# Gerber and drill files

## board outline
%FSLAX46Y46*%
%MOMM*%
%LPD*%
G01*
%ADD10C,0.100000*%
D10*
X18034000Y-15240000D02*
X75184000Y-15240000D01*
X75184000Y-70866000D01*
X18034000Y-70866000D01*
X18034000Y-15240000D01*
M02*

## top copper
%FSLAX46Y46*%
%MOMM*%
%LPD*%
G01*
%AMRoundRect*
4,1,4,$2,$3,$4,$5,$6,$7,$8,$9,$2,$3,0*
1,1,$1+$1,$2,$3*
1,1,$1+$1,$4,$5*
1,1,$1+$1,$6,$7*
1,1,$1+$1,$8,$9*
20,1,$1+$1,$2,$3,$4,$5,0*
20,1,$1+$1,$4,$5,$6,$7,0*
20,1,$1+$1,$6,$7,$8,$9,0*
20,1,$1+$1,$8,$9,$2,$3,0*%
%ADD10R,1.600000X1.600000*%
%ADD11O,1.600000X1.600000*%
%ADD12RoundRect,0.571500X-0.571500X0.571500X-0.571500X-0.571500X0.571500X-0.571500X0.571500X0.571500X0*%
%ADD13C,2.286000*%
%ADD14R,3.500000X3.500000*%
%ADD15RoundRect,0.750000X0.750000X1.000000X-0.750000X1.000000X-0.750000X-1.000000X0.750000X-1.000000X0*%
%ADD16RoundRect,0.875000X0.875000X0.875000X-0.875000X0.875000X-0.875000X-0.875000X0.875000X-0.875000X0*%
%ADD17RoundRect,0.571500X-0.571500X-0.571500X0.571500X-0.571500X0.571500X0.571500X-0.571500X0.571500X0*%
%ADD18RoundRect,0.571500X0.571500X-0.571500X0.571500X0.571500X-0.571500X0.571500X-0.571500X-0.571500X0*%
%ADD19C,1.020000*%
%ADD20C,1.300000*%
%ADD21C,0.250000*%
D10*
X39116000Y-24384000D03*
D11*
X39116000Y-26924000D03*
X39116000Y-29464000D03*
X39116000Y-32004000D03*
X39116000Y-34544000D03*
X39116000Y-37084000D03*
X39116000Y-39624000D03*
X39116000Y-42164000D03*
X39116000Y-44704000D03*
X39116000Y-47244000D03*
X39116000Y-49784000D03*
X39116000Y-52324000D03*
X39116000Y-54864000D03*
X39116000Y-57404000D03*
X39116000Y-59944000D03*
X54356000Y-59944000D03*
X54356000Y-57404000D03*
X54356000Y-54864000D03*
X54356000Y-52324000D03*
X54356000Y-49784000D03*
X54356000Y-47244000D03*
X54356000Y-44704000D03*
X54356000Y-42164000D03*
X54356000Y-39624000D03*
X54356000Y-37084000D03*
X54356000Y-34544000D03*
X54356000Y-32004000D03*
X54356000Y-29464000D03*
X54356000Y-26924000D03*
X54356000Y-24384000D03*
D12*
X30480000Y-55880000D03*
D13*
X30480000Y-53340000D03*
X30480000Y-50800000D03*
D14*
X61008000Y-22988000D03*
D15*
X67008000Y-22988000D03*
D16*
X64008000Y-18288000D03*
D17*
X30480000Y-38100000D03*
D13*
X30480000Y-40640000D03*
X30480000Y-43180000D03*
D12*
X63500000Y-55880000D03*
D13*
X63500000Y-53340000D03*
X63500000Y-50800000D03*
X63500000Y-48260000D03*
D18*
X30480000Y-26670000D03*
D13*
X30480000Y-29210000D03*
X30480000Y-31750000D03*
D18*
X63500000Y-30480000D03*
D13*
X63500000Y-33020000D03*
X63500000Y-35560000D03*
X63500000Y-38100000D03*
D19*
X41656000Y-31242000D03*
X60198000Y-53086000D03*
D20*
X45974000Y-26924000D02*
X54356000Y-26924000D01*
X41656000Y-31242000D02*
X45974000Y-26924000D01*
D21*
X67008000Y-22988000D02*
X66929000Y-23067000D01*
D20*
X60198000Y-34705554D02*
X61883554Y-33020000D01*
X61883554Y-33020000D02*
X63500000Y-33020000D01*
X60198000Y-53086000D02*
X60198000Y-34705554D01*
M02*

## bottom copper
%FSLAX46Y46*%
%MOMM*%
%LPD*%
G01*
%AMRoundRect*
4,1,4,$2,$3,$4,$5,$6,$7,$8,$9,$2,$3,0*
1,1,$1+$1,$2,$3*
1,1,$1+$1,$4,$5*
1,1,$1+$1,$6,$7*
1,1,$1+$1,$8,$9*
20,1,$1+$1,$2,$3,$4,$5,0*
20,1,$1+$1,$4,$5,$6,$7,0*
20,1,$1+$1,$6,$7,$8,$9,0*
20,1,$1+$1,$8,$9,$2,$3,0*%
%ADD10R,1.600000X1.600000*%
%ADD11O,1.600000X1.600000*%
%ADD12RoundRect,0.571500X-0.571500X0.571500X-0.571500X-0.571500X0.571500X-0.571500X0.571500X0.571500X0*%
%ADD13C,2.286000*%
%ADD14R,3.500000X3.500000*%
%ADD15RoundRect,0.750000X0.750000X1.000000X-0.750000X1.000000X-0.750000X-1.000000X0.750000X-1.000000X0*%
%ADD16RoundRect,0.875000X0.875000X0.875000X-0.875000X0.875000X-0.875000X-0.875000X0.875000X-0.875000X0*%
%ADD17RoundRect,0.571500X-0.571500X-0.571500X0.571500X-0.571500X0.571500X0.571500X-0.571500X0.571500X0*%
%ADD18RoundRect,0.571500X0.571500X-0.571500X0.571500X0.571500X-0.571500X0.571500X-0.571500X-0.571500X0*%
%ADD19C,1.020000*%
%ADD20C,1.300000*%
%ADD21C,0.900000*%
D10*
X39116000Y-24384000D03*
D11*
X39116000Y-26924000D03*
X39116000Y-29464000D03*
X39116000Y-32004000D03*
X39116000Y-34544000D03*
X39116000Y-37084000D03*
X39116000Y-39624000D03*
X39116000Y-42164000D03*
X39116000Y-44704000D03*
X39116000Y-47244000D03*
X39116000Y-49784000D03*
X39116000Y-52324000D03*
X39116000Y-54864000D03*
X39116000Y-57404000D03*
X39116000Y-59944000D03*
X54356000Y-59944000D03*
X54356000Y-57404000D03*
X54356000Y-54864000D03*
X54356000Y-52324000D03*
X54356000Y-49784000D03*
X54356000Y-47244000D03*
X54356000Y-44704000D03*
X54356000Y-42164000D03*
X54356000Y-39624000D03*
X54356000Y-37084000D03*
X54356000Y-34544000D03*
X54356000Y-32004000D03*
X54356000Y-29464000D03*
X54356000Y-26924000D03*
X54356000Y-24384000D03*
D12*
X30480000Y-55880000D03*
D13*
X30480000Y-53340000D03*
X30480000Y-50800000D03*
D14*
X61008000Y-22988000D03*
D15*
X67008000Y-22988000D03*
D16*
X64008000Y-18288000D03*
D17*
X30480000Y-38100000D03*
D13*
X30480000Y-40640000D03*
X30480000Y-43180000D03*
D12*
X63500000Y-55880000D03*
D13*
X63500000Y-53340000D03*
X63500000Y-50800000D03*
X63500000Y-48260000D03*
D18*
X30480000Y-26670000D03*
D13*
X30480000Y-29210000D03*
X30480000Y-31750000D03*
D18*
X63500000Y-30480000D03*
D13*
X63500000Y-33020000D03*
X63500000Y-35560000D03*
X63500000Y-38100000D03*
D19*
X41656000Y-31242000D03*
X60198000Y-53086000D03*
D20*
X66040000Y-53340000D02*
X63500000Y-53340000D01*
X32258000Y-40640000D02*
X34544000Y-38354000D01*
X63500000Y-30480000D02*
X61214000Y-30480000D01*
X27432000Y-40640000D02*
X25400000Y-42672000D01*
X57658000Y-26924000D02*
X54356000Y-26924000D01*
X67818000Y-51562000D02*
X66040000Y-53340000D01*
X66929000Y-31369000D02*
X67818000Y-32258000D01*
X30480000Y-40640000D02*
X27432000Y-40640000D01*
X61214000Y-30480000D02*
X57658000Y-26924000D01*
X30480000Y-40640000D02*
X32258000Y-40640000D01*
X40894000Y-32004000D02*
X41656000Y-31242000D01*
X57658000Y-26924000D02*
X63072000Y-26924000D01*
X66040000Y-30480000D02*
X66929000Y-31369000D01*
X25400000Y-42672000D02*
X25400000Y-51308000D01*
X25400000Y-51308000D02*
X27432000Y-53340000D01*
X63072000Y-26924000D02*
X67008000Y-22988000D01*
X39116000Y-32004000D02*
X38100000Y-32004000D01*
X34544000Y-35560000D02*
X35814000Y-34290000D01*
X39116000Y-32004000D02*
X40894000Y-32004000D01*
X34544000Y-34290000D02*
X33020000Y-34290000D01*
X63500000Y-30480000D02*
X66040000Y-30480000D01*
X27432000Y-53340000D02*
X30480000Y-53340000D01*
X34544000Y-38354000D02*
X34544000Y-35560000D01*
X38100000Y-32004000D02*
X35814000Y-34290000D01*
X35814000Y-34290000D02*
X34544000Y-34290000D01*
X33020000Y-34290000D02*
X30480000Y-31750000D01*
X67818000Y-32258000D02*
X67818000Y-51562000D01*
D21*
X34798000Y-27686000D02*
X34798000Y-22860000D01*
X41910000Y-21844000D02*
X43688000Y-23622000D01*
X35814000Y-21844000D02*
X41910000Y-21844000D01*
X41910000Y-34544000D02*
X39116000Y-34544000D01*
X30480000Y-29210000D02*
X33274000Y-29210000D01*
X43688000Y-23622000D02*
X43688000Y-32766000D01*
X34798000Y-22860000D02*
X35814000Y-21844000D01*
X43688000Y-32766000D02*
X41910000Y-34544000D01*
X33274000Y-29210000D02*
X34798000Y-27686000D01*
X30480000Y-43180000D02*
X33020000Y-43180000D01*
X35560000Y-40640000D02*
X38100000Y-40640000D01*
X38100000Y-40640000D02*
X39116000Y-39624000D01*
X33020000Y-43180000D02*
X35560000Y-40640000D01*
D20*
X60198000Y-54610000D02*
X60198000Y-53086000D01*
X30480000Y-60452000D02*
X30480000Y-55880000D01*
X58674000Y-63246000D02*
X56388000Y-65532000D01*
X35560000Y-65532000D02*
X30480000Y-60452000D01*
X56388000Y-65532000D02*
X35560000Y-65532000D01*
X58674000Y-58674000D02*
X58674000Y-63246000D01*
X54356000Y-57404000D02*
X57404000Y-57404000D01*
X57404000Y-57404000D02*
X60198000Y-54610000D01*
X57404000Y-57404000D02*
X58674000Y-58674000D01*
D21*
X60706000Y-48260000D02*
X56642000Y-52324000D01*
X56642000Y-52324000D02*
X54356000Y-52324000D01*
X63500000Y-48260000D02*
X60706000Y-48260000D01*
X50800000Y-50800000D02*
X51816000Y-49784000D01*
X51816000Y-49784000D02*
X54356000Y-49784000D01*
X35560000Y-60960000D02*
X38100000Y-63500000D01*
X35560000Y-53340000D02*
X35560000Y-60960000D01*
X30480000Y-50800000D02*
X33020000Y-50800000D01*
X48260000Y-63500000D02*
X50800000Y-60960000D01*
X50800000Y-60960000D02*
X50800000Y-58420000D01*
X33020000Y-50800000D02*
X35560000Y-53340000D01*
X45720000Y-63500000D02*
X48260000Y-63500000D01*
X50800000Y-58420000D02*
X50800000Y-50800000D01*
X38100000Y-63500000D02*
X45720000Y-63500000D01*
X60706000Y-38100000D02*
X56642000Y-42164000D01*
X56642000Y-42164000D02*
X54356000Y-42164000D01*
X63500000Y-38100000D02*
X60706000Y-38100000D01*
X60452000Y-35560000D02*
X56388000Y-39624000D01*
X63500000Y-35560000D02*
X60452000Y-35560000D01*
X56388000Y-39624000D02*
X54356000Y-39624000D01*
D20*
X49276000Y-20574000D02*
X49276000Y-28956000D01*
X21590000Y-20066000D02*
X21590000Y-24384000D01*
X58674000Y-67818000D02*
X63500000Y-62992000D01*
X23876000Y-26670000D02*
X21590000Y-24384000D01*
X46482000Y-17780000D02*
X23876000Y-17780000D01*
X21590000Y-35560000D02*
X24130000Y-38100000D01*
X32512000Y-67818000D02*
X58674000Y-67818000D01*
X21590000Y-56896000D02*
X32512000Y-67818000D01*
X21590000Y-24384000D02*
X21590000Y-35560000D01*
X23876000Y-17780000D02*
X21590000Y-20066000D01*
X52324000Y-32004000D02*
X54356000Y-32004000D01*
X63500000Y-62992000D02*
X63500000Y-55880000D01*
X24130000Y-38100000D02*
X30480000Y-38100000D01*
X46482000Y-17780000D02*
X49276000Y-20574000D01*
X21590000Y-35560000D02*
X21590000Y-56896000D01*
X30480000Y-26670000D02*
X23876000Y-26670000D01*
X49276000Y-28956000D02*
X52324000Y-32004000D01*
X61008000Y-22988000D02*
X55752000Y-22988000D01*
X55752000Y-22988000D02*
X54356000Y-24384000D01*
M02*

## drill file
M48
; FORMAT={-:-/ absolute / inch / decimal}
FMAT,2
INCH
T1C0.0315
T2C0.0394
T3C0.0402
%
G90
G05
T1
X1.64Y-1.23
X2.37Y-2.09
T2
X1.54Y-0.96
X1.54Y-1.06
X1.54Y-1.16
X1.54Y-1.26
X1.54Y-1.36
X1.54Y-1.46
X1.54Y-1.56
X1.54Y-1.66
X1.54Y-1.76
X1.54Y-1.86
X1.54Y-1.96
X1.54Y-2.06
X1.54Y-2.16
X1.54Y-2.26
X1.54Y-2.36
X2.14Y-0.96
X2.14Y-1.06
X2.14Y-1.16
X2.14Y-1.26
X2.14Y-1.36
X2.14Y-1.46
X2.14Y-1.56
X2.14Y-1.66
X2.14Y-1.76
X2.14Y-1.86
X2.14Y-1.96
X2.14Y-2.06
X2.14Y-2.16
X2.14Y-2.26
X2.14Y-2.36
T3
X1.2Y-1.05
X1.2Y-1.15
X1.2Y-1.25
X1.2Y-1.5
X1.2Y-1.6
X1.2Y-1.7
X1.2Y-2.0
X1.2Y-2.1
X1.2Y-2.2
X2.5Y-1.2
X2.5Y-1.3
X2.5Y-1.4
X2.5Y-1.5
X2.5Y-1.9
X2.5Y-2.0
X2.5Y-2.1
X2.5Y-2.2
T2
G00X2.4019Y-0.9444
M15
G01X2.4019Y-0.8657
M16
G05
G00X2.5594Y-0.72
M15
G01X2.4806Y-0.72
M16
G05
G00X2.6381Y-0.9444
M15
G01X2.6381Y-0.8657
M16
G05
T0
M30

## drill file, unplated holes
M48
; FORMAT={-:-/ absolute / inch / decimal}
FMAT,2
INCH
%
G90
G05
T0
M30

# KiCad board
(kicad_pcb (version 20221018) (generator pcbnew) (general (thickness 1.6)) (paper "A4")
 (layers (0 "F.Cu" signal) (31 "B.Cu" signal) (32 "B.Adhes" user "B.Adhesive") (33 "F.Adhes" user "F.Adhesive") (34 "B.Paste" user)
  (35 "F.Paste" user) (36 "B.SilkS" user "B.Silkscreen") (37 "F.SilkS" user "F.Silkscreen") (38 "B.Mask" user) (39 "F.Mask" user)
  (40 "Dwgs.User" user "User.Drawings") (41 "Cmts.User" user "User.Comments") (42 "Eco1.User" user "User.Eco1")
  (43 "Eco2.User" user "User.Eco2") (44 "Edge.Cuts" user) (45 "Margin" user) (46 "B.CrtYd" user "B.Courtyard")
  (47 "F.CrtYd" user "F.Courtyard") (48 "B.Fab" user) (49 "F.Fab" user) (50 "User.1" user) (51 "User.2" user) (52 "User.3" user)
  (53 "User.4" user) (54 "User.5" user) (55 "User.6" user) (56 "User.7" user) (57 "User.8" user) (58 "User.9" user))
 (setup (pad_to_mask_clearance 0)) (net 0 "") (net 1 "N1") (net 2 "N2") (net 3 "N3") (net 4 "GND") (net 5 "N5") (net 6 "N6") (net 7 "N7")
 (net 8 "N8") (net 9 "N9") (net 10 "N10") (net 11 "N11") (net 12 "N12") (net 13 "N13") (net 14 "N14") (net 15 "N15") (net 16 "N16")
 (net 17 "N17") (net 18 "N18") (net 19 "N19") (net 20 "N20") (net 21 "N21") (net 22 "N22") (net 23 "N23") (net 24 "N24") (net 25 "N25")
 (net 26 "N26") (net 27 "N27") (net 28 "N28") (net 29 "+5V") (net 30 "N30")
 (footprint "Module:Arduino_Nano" (layer "F.Cu") (at 39.116 24.384)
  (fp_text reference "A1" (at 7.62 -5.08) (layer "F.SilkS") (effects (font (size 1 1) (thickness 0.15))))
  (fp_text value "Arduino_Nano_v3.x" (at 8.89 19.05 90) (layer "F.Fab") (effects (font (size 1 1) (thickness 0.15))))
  (pad "1" thru_hole rect (at 0 0) (size 1.6 1.6) (drill 1) (layers "*.Cu" "*.Mask") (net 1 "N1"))
  (pad "2" thru_hole oval (at 0 2.54) (size 1.6 1.6) (drill 1) (layers "*.Cu" "*.Mask") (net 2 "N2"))
  (pad "3" thru_hole oval (at 0 5.08) (size 1.6 1.6) (drill 1) (layers "*.Cu" "*.Mask") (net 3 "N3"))
  (pad "4" thru_hole oval (at 0 7.62) (size 1.6 1.6) (drill 1) (layers "*.Cu" "*.Mask") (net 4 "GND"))
  (pad "5" thru_hole oval (at 0 10.16) (size 1.6 1.6) (drill 1) (layers "*.Cu" "*.Mask") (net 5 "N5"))
  (pad "6" thru_hole oval (at 0 12.7) (size 1.6 1.6) (drill 1) (layers "*.Cu" "*.Mask") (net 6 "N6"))
  (pad "7" thru_hole oval (at 0 15.24) (size 1.6 1.6) (drill 1) (layers "*.Cu" "*.Mask") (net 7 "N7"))
  (pad "8" thru_hole oval (at 0 17.78) (size 1.6 1.6) (drill 1) (layers "*.Cu" "*.Mask") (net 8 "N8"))
  (pad "9" thru_hole oval (at 0 20.32) (size 1.6 1.6) (drill 1) (layers "*.Cu" "*.Mask") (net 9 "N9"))
  (pad "10" thru_hole oval (at 0 22.86) (size 1.6 1.6) (drill 1) (layers "*.Cu" "*.Mask") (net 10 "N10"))
  (pad "11" thru_hole oval (at 0 25.4) (size 1.6 1.6) (drill 1) (layers "*.Cu" "*.Mask") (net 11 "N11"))
  (pad "12" thru_hole oval (at 0 27.94) (size 1.6 1.6) (drill 1) (layers "*.Cu" "*.Mask") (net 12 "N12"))
  (pad "13" thru_hole oval (at 0 30.48) (size 1.6 1.6) (drill 1) (layers "*.Cu" "*.Mask") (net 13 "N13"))
  (pad "14" thru_hole oval (at 0 33.02) (size 1.6 1.6) (drill 1) (layers "*.Cu" "*.Mask") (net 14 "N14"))
  (pad "15" thru_hole oval (at 0 35.56) (size 1.6 1.6) (drill 1) (layers "*.Cu" "*.Mask") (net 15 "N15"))
  (pad "16" thru_hole oval (at 15.24 35.56) (size 1.6 1.6) (drill 1) (layers "*.Cu" "*.Mask") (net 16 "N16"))
  (pad "17" thru_hole oval (at 15.24 33.02) (size 1.6 1.6) (drill 1) (layers "*.Cu" "*.Mask") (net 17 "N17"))
  (pad "18" thru_hole oval (at 15.24 30.48) (size 1.6 1.6) (drill 1) (layers "*.Cu" "*.Mask") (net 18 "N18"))
  (pad "19" thru_hole oval (at 15.24 27.94) (size 1.6 1.6) (drill 1) (layers "*.Cu" "*.Mask") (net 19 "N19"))
  (pad "20" thru_hole oval (at 15.24 25.4) (size 1.6 1.6) (drill 1) (layers "*.Cu" "*.Mask") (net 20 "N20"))
  (pad "21" thru_hole oval (at 15.24 22.86) (size 1.6 1.6) (drill 1) (layers "*.Cu" "*.Mask") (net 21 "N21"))
  (pad "22" thru_hole oval (at 15.24 20.32) (size 1.6 1.6) (drill 1) (layers "*.Cu" "*.Mask") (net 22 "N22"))
  (pad "23" thru_hole oval (at 15.24 17.78) (size 1.6 1.6) (drill 1) (layers "*.Cu" "*.Mask") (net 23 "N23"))
  (pad "24" thru_hole oval (at 15.24 15.24) (size 1.6 1.6) (drill 1) (layers "*.Cu" "*.Mask") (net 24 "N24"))
  (pad "25" thru_hole oval (at 15.24 12.7) (size 1.6 1.6) (drill 1) (layers "*.Cu" "*.Mask") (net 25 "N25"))
  (pad "26" thru_hole oval (at 15.24 10.16) (size 1.6 1.6) (drill 1) (layers "*.Cu" "*.Mask") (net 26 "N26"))
  (pad "27" thru_hole oval (at 15.24 7.62) (size 1.6 1.6) (drill 1) (layers "*.Cu" "*.Mask") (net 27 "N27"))
  (pad "28" thru_hole oval (at 15.24 5.08) (size 1.6 1.6) (drill 1) (layers "*.Cu" "*.Mask") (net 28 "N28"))
  (pad "29" thru_hole oval (at 15.24 2.54) (size 1.6 1.6) (drill 1) (layers "*.Cu" "*.Mask") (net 4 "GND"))
  (pad "30" thru_hole oval (at 15.24 0) (size 1.6 1.6) (drill 1) (layers "*.Cu" "*.Mask") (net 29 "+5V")))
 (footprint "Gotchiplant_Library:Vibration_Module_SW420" (layer "F.Cu") (at 30.48 53.34 180)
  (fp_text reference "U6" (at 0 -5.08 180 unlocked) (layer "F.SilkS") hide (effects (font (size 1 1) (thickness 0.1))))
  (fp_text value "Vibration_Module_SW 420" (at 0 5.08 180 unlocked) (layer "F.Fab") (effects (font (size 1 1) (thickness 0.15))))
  (pad "1" thru_hole roundrect (at 0 -2.54 270) (size 2.286 2.286) (drill 1.02) (layers "*.Cu" "*.Mask") (roundrect_rratio 0.25)
   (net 17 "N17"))
  (pad "2" thru_hole circle (at 0 0 270) (size 2.286 2.286) (drill 1.02) (layers "*.Cu" "*.Mask") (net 4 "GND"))
  (pad "3" thru_hole circle (at 0 2.54 270) (size 2.286 2.286) (drill 1.02) (layers "*.Cu" "*.Mask") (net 20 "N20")))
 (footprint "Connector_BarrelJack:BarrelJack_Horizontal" (layer "F.Cu") (at 61.008 22.988 180)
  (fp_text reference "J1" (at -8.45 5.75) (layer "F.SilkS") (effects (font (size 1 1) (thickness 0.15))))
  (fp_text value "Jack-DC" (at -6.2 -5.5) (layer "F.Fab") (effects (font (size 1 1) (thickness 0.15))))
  (pad "1" thru_hole rect (at 0 0 180) (size 3.5 3.5) (drill oval 1 3) (layers "*.Cu" "*.Mask") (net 29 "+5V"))
  (pad "2" thru_hole roundrect (at -6 0 180) (size 3 3.5) (drill oval 1 3) (layers "*.Cu" "*.Mask") (roundrect_rratio 0.25) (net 4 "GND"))
  (pad "3" thru_hole roundrect (at -3 4.7 180) (size 3.5 3.5) (drill oval 3 1) (layers "*.Cu" "*.Mask") (roundrect_rratio 0.25)))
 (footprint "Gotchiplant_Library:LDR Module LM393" (layer "F.Cu") (at 30.48 40.64)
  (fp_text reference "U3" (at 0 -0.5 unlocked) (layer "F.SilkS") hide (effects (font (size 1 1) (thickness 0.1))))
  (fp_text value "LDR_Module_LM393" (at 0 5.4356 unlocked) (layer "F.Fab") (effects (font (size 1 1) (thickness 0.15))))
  (pad "1" thru_hole roundrect (at 0 -2.54) (size 2.286 2.286) (drill 1.02) (layers "*.Cu" "*.Mask") (roundrect_rratio 0.25) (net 27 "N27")
   (thermal_bridge_angle 45))
  (pad "2" thru_hole circle (at 0 0) (size 2.286 2.286) (drill 1.02) (layers "*.Cu" "*.Mask") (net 4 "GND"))
  (pad "3" thru_hole circle (at 0 2.54) (size 2.286 2.286) (drill 1.02) (layers "*.Cu" "*.Mask") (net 7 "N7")))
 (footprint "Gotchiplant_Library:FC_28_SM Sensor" (layer "F.Cu") (at 63.5 52.07 180)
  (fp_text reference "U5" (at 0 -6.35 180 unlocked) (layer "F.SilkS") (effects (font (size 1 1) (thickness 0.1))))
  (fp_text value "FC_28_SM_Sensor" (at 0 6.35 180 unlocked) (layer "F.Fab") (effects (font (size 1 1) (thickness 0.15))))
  (pad "1" thru_hole roundrect (at 0 -3.81 270) (size 2.286 2.286) (drill 1.02) (layers "*.Cu" "*.Mask") (roundrect_rratio 0.25)
   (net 27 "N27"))
  (pad "2" thru_hole circle (at 0 -1.27 270) (size 2.286 2.286) (drill 1.02) (layers "*.Cu" "*.Mask") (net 4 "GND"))
  (pad "3" thru_hole circle (at 0 1.27 270) (size 2.286 2.286) (drill 1.02) (layers "*.Cu" "*.Mask") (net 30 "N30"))
  (pad "4" thru_hole circle (at 0 3.81 270) (size 2.286 2.286) (drill 1.02) (layers "*.Cu" "*.Mask") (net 19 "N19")))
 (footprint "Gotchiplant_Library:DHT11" (layer "F.Cu") (at 30.48 29.21)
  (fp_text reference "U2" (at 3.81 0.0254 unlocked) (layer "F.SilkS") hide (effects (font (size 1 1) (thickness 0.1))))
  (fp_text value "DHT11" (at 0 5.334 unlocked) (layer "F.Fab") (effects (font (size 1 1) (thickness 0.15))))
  (pad "1" thru_hole roundrect (at 0 -2.54 90) (size 2.286 2.286) (drill 1.02) (layers "*.Cu" "*.Mask") (roundrect_rratio 0.25)
   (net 27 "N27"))
  (pad "2" thru_hole circle (at 0 0) (size 2.286 2.286) (drill 1.02) (layers "*.Cu" "*.Mask") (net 5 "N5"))
  (pad "3" thru_hole circle (at 0 2.54) (size 2.286 2.286) (drill 1.02) (layers "*.Cu" "*.Mask") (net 4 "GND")))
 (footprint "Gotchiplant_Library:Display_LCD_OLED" (layer "F.Cu") (at 63.5 34.29)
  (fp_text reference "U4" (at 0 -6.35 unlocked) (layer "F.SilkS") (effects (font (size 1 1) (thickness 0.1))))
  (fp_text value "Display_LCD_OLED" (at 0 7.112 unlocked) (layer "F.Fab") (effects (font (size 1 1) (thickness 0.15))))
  (pad "1" thru_hole roundrect (at 0 -3.81 90) (size 2.286 2.286) (drill 1.02) (layers "*.Cu" "*.Mask") (roundrect_rratio 0.25)
   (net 4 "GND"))
  (pad "2" thru_hole circle (at 0 -1.27 90) (size 2.286 2.286) (drill 1.02) (layers "*.Cu" "*.Mask") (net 17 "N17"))
  (pad "3" thru_hole circle (at 0 1.27 90) (size 2.286 2.286) (drill 1.02) (layers "*.Cu" "*.Mask") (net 24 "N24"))
  (pad "4" thru_hole circle (at 0 3.81 90) (size 2.286 2.286) (drill 1.02) (layers "*.Cu" "*.Mask") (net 23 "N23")))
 (gr_rect (start 18.034 15.24) (end 75.184 70.866) (stroke (width 0.1) (type default)) (fill none) (layer "Edge.Cuts"))
 (segment (start 45.974 26.924) (end 54.356 26.924) (width 1.3) (layer "F.Cu") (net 4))
 (segment (start 41.656 31.242) (end 45.974 26.924) (width 1.3) (layer "F.Cu") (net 4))
 (segment (start 67.008 22.988) (end 66.929 23.067) (width 0.25) (layer "F.Cu") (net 4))
 (via (at 41.656 31.242) (size 1.02) (drill 0.8) (layers "F.Cu" "B.Cu") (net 4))
 (segment (start 66.04 53.34) (end 63.5 53.34) (width 1.3) (layer "B.Cu") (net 4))
 (segment (start 32.258 40.64) (end 34.544 38.354) (width 1.3) (layer "B.Cu") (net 4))
 (segment (start 63.5 30.48) (end 61.214 30.48) (width 1.3) (layer "B.Cu") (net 4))
 (segment (start 27.432 40.64) (end 25.4 42.672) (width 1.3) (layer "B.Cu") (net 4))
 (segment (start 57.658 26.924) (end 54.356 26.924) (width 1.3) (layer "B.Cu") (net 4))
 (segment (start 67.818 51.562) (end 66.04 53.34) (width 1.3) (layer "B.Cu") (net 4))
 (segment (start 66.929 31.369) (end 67.818 32.258) (width 1.3) (layer "B.Cu") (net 4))
 (segment (start 30.48 40.64) (end 27.432 40.64) (width 1.3) (layer "B.Cu") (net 4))
 (segment (start 61.214 30.48) (end 57.658 26.924) (width 1.3) (layer "B.Cu") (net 4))
 (segment (start 30.48 40.64) (end 32.258 40.64) (width 1.3) (layer "B.Cu") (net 4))
 (segment (start 40.894 32.004) (end 41.656 31.242) (width 1.3) (layer "B.Cu") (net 4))
 (segment (start 57.658 26.924) (end 63.072 26.924) (width 1.3) (layer "B.Cu") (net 4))
 (segment (start 66.04 30.48) (end 66.929 31.369) (width 1.3) (layer "B.Cu") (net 4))
 (segment (start 25.4 42.672) (end 25.4 51.308) (width 1.3) (layer "B.Cu") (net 4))
 (segment (start 25.4 51.308) (end 27.432 53.34) (width 1.3) (layer "B.Cu") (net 4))
 (segment (start 63.072 26.924) (end 67.008 22.988) (width 1.3) (layer "B.Cu") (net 4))
 (segment (start 39.116 32.004) (end 38.1 32.004) (width 1.3) (layer "B.Cu") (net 4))
 (segment (start 34.544 35.56) (end 35.814 34.29) (width 1.3) (layer "B.Cu") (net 4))
 (segment (start 39.116 32.004) (end 40.894 32.004) (width 1.3) (layer "B.Cu") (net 4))
 (segment (start 34.544 34.29) (end 33.02 34.29) (width 1.3) (layer "B.Cu") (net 4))
 (segment (start 63.5 30.48) (end 66.04 30.48) (width 1.3) (layer "B.Cu") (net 4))
 (segment (start 27.432 53.34) (end 30.48 53.34) (width 1.3) (layer "B.Cu") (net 4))
 (segment (start 34.544 38.354) (end 34.544 35.56) (width 1.3) (layer "B.Cu") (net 4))
 (segment (start 38.1 32.004) (end 35.814 34.29) (width 1.3) (layer "B.Cu") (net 4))
 (segment (start 35.814 34.29) (end 34.544 34.29) (width 1.3) (layer "B.Cu") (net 4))
 (segment (start 33.02 34.29) (end 30.48 31.75) (width 1.3) (layer "B.Cu") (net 4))
 (segment (start 67.818 32.258) (end 67.818 51.562) (width 1.3) (layer "B.Cu") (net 4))
 (segment (start 34.798 27.686) (end 34.798 22.86) (width 0.9) (layer "B.Cu") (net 5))
 (segment (start 41.91 21.844) (end 43.688 23.622) (width 0.9) (layer "B.Cu") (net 5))
 (segment (start 35.814 21.844) (end 41.91 21.844) (width 0.9) (layer "B.Cu") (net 5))
 (segment (start 41.91 34.544) (end 39.116 34.544) (width 0.9) (layer "B.Cu") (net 5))
 (segment (start 30.48 29.21) (end 33.274 29.21) (width 0.9) (layer "B.Cu") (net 5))
 (segment (start 43.688 23.622) (end 43.688 32.766) (width 0.9) (layer "B.Cu") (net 5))
 (segment (start 34.798 22.86) (end 35.814 21.844) (width 0.9) (layer "B.Cu") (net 5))
 (segment (start 43.688 32.766) (end 41.91 34.544) (width 0.9) (layer "B.Cu") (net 5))
 (segment (start 33.274 29.21) (end 34.798 27.686) (width 0.9) (layer "B.Cu") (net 5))
 (segment (start 30.48 43.18) (end 33.02 43.18) (width 0.9) (layer "B.Cu") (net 7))
 (segment (start 35.56 40.64) (end 38.1 40.64) (width 0.9) (layer "B.Cu") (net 7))
 (segment (start 38.1 40.64) (end 39.116 39.624) (width 0.9) (layer "B.Cu") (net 7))
 (segment (start 33.02 43.18) (end 35.56 40.64) (width 0.9) (layer "B.Cu") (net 7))
 (segment (start 60.198 34.705554) (end 61.883554 33.02) (width 1.3) (layer "F.Cu") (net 17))
 (segment (start 61.883554 33.02) (end 63.5 33.02) (width 1.3) (layer "F.Cu") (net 17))
 (segment (start 60.198 53.086) (end 60.198 34.705554) (width 1.3) (layer "F.Cu") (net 17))
 (via (at 60.198 53.086) (size 1.02) (drill 0.8) (layers "F.Cu" "B.Cu") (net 17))
 (segment (start 60.198 54.61) (end 60.198 53.086) (width 1.3) (layer "B.Cu") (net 17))
 (segment (start 30.48 60.452) (end 30.48 55.88) (width 1.3) (layer "B.Cu") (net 17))
 (segment (start 58.674 63.246) (end 56.388 65.532) (width 1.3) (layer "B.Cu") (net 17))
 (segment (start 35.56 65.532) (end 30.48 60.452) (width 1.3) (layer "B.Cu") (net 17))
 (segment (start 56.388 65.532) (end 35.56 65.532) (width 1.3) (layer "B.Cu") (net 17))
 (segment (start 58.674 58.674) (end 58.674 63.246) (width 1.3) (layer "B.Cu") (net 17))
 (segment (start 54.356 57.404) (end 57.404 57.404) (width 1.3) (layer "B.Cu") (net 17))
 (segment (start 57.404 57.404) (end 60.198 54.61) (width 1.3) (layer "B.Cu") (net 17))
 (segment (start 57.404 57.404) (end 58.674 58.674) (width 1.3) (layer "B.Cu") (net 17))
 (segment (start 60.706 48.26) (end 56.642 52.324) (width 0.9) (layer "B.Cu") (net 19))
 (segment (start 56.642 52.324) (end 54.356 52.324) (width 0.9) (layer "B.Cu") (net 19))
 (segment (start 63.5 48.26) (end 60.706 48.26) (width 0.9) (layer "B.Cu") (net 19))
 (segment (start 50.8 50.8) (end 51.816 49.784) (width 0.9) (layer "B.Cu") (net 20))
 (segment (start 51.816 49.784) (end 54.356 49.784) (width 0.9) (layer "B.Cu") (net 20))
 (segment (start 35.56 60.96) (end 38.1 63.5) (width 0.9) (layer "B.Cu") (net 20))
 (segment (start 35.56 53.34) (end 35.56 60.96) (width 0.9) (layer "B.Cu") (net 20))
 (segment (start 30.48 50.8) (end 33.02 50.8) (width 0.9) (layer "B.Cu") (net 20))
 (segment (start 48.26 63.5) (end 50.8 60.96) (width 0.9) (layer "B.Cu") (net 20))
 (segment (start 50.8 60.96) (end 50.8 58.42) (width 0.9) (layer "B.Cu") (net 20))
 (segment (start 33.02 50.8) (end 35.56 53.34) (width 0.9) (layer "B.Cu") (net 20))
 (segment (start 45.72 63.5) (end 48.26 63.5) (width 0.9) (layer "B.Cu") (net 20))
 (segment (start 50.8 58.42) (end 50.8 50.8) (width 0.9) (layer "B.Cu") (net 20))
 (segment (start 38.1 63.5) (end 45.72 63.5) (width 0.9) (layer "B.Cu") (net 20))
 (segment (start 60.706 38.1) (end 56.642 42.164) (width 0.9) (layer "B.Cu") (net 23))
 (segment (start 56.642 42.164) (end 54.356 42.164) (width 0.9) (layer "B.Cu") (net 23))
 (segment (start 63.5 38.1) (end 60.706 38.1) (width 0.9) (layer "B.Cu") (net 23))
 (segment (start 60.452 35.56) (end 56.388 39.624) (width 0.9) (layer "B.Cu") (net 24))
 (segment (start 63.5 35.56) (end 60.452 35.56) (width 0.9) (layer "B.Cu") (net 24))
 (segment (start 56.388 39.624) (end 54.356 39.624) (width 0.9) (layer "B.Cu") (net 24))
 (segment (start 49.276 20.574) (end 49.276 28.956) (width 1.3) (layer "B.Cu") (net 27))
 (segment (start 21.59 20.066) (end 21.59 24.384) (width 1.3) (layer "B.Cu") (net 27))
 (segment (start 58.674 67.818) (end 63.5 62.992) (width 1.3) (layer "B.Cu") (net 27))
 (segment (start 23.876 26.67) (end 21.59 24.384) (width 1.3) (layer "B.Cu") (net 27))
 (segment (start 46.482 17.78) (end 23.876 17.78) (width 1.3) (layer "B.Cu") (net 27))
 (segment (start 21.59 35.56) (end 24.13 38.1) (width 1.3) (layer "B.Cu") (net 27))
 (segment (start 32.512 67.818) (end 58.674 67.818) (width 1.3) (layer "B.Cu") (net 27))
 (segment (start 21.59 56.896) (end 32.512 67.818) (width 1.3) (layer "B.Cu") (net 27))
 (segment (start 21.59 24.384) (end 21.59 35.56) (width 1.3) (layer "B.Cu") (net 27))
 (segment (start 23.876 17.78) (end 21.59 20.066) (width 1.3) (layer "B.Cu") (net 27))
 (segment (start 52.324 32.004) (end 54.356 32.004) (width 1.3) (layer "B.Cu") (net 27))
 (segment (start 63.5 62.992) (end 63.5 55.88) (width 1.3) (layer "B.Cu") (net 27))
 (segment (start 24.13 38.1) (end 30.48 38.1) (width 1.3) (layer "B.Cu") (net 27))
 (segment (start 46.482 17.78) (end 49.276 20.574) (width 1.3) (layer "B.Cu") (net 27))
 (segment (start 21.59 35.56) (end 21.59 56.896) (width 1.3) (layer "B.Cu") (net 27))
 (segment (start 30.48 26.67) (end 23.876 26.67) (width 1.3) (layer "B.Cu") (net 27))
 (segment (start 49.276 28.956) (end 52.324 32.004) (width 1.3) (layer "B.Cu") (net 27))
 (segment (start 61.008 22.988) (end 55.752 22.988) (width 1.3) (layer "B.Cu") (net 29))
 (segment (start 55.752 22.988) (end 54.356 24.384) (width 1.3) (layer "B.Cu") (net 29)))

